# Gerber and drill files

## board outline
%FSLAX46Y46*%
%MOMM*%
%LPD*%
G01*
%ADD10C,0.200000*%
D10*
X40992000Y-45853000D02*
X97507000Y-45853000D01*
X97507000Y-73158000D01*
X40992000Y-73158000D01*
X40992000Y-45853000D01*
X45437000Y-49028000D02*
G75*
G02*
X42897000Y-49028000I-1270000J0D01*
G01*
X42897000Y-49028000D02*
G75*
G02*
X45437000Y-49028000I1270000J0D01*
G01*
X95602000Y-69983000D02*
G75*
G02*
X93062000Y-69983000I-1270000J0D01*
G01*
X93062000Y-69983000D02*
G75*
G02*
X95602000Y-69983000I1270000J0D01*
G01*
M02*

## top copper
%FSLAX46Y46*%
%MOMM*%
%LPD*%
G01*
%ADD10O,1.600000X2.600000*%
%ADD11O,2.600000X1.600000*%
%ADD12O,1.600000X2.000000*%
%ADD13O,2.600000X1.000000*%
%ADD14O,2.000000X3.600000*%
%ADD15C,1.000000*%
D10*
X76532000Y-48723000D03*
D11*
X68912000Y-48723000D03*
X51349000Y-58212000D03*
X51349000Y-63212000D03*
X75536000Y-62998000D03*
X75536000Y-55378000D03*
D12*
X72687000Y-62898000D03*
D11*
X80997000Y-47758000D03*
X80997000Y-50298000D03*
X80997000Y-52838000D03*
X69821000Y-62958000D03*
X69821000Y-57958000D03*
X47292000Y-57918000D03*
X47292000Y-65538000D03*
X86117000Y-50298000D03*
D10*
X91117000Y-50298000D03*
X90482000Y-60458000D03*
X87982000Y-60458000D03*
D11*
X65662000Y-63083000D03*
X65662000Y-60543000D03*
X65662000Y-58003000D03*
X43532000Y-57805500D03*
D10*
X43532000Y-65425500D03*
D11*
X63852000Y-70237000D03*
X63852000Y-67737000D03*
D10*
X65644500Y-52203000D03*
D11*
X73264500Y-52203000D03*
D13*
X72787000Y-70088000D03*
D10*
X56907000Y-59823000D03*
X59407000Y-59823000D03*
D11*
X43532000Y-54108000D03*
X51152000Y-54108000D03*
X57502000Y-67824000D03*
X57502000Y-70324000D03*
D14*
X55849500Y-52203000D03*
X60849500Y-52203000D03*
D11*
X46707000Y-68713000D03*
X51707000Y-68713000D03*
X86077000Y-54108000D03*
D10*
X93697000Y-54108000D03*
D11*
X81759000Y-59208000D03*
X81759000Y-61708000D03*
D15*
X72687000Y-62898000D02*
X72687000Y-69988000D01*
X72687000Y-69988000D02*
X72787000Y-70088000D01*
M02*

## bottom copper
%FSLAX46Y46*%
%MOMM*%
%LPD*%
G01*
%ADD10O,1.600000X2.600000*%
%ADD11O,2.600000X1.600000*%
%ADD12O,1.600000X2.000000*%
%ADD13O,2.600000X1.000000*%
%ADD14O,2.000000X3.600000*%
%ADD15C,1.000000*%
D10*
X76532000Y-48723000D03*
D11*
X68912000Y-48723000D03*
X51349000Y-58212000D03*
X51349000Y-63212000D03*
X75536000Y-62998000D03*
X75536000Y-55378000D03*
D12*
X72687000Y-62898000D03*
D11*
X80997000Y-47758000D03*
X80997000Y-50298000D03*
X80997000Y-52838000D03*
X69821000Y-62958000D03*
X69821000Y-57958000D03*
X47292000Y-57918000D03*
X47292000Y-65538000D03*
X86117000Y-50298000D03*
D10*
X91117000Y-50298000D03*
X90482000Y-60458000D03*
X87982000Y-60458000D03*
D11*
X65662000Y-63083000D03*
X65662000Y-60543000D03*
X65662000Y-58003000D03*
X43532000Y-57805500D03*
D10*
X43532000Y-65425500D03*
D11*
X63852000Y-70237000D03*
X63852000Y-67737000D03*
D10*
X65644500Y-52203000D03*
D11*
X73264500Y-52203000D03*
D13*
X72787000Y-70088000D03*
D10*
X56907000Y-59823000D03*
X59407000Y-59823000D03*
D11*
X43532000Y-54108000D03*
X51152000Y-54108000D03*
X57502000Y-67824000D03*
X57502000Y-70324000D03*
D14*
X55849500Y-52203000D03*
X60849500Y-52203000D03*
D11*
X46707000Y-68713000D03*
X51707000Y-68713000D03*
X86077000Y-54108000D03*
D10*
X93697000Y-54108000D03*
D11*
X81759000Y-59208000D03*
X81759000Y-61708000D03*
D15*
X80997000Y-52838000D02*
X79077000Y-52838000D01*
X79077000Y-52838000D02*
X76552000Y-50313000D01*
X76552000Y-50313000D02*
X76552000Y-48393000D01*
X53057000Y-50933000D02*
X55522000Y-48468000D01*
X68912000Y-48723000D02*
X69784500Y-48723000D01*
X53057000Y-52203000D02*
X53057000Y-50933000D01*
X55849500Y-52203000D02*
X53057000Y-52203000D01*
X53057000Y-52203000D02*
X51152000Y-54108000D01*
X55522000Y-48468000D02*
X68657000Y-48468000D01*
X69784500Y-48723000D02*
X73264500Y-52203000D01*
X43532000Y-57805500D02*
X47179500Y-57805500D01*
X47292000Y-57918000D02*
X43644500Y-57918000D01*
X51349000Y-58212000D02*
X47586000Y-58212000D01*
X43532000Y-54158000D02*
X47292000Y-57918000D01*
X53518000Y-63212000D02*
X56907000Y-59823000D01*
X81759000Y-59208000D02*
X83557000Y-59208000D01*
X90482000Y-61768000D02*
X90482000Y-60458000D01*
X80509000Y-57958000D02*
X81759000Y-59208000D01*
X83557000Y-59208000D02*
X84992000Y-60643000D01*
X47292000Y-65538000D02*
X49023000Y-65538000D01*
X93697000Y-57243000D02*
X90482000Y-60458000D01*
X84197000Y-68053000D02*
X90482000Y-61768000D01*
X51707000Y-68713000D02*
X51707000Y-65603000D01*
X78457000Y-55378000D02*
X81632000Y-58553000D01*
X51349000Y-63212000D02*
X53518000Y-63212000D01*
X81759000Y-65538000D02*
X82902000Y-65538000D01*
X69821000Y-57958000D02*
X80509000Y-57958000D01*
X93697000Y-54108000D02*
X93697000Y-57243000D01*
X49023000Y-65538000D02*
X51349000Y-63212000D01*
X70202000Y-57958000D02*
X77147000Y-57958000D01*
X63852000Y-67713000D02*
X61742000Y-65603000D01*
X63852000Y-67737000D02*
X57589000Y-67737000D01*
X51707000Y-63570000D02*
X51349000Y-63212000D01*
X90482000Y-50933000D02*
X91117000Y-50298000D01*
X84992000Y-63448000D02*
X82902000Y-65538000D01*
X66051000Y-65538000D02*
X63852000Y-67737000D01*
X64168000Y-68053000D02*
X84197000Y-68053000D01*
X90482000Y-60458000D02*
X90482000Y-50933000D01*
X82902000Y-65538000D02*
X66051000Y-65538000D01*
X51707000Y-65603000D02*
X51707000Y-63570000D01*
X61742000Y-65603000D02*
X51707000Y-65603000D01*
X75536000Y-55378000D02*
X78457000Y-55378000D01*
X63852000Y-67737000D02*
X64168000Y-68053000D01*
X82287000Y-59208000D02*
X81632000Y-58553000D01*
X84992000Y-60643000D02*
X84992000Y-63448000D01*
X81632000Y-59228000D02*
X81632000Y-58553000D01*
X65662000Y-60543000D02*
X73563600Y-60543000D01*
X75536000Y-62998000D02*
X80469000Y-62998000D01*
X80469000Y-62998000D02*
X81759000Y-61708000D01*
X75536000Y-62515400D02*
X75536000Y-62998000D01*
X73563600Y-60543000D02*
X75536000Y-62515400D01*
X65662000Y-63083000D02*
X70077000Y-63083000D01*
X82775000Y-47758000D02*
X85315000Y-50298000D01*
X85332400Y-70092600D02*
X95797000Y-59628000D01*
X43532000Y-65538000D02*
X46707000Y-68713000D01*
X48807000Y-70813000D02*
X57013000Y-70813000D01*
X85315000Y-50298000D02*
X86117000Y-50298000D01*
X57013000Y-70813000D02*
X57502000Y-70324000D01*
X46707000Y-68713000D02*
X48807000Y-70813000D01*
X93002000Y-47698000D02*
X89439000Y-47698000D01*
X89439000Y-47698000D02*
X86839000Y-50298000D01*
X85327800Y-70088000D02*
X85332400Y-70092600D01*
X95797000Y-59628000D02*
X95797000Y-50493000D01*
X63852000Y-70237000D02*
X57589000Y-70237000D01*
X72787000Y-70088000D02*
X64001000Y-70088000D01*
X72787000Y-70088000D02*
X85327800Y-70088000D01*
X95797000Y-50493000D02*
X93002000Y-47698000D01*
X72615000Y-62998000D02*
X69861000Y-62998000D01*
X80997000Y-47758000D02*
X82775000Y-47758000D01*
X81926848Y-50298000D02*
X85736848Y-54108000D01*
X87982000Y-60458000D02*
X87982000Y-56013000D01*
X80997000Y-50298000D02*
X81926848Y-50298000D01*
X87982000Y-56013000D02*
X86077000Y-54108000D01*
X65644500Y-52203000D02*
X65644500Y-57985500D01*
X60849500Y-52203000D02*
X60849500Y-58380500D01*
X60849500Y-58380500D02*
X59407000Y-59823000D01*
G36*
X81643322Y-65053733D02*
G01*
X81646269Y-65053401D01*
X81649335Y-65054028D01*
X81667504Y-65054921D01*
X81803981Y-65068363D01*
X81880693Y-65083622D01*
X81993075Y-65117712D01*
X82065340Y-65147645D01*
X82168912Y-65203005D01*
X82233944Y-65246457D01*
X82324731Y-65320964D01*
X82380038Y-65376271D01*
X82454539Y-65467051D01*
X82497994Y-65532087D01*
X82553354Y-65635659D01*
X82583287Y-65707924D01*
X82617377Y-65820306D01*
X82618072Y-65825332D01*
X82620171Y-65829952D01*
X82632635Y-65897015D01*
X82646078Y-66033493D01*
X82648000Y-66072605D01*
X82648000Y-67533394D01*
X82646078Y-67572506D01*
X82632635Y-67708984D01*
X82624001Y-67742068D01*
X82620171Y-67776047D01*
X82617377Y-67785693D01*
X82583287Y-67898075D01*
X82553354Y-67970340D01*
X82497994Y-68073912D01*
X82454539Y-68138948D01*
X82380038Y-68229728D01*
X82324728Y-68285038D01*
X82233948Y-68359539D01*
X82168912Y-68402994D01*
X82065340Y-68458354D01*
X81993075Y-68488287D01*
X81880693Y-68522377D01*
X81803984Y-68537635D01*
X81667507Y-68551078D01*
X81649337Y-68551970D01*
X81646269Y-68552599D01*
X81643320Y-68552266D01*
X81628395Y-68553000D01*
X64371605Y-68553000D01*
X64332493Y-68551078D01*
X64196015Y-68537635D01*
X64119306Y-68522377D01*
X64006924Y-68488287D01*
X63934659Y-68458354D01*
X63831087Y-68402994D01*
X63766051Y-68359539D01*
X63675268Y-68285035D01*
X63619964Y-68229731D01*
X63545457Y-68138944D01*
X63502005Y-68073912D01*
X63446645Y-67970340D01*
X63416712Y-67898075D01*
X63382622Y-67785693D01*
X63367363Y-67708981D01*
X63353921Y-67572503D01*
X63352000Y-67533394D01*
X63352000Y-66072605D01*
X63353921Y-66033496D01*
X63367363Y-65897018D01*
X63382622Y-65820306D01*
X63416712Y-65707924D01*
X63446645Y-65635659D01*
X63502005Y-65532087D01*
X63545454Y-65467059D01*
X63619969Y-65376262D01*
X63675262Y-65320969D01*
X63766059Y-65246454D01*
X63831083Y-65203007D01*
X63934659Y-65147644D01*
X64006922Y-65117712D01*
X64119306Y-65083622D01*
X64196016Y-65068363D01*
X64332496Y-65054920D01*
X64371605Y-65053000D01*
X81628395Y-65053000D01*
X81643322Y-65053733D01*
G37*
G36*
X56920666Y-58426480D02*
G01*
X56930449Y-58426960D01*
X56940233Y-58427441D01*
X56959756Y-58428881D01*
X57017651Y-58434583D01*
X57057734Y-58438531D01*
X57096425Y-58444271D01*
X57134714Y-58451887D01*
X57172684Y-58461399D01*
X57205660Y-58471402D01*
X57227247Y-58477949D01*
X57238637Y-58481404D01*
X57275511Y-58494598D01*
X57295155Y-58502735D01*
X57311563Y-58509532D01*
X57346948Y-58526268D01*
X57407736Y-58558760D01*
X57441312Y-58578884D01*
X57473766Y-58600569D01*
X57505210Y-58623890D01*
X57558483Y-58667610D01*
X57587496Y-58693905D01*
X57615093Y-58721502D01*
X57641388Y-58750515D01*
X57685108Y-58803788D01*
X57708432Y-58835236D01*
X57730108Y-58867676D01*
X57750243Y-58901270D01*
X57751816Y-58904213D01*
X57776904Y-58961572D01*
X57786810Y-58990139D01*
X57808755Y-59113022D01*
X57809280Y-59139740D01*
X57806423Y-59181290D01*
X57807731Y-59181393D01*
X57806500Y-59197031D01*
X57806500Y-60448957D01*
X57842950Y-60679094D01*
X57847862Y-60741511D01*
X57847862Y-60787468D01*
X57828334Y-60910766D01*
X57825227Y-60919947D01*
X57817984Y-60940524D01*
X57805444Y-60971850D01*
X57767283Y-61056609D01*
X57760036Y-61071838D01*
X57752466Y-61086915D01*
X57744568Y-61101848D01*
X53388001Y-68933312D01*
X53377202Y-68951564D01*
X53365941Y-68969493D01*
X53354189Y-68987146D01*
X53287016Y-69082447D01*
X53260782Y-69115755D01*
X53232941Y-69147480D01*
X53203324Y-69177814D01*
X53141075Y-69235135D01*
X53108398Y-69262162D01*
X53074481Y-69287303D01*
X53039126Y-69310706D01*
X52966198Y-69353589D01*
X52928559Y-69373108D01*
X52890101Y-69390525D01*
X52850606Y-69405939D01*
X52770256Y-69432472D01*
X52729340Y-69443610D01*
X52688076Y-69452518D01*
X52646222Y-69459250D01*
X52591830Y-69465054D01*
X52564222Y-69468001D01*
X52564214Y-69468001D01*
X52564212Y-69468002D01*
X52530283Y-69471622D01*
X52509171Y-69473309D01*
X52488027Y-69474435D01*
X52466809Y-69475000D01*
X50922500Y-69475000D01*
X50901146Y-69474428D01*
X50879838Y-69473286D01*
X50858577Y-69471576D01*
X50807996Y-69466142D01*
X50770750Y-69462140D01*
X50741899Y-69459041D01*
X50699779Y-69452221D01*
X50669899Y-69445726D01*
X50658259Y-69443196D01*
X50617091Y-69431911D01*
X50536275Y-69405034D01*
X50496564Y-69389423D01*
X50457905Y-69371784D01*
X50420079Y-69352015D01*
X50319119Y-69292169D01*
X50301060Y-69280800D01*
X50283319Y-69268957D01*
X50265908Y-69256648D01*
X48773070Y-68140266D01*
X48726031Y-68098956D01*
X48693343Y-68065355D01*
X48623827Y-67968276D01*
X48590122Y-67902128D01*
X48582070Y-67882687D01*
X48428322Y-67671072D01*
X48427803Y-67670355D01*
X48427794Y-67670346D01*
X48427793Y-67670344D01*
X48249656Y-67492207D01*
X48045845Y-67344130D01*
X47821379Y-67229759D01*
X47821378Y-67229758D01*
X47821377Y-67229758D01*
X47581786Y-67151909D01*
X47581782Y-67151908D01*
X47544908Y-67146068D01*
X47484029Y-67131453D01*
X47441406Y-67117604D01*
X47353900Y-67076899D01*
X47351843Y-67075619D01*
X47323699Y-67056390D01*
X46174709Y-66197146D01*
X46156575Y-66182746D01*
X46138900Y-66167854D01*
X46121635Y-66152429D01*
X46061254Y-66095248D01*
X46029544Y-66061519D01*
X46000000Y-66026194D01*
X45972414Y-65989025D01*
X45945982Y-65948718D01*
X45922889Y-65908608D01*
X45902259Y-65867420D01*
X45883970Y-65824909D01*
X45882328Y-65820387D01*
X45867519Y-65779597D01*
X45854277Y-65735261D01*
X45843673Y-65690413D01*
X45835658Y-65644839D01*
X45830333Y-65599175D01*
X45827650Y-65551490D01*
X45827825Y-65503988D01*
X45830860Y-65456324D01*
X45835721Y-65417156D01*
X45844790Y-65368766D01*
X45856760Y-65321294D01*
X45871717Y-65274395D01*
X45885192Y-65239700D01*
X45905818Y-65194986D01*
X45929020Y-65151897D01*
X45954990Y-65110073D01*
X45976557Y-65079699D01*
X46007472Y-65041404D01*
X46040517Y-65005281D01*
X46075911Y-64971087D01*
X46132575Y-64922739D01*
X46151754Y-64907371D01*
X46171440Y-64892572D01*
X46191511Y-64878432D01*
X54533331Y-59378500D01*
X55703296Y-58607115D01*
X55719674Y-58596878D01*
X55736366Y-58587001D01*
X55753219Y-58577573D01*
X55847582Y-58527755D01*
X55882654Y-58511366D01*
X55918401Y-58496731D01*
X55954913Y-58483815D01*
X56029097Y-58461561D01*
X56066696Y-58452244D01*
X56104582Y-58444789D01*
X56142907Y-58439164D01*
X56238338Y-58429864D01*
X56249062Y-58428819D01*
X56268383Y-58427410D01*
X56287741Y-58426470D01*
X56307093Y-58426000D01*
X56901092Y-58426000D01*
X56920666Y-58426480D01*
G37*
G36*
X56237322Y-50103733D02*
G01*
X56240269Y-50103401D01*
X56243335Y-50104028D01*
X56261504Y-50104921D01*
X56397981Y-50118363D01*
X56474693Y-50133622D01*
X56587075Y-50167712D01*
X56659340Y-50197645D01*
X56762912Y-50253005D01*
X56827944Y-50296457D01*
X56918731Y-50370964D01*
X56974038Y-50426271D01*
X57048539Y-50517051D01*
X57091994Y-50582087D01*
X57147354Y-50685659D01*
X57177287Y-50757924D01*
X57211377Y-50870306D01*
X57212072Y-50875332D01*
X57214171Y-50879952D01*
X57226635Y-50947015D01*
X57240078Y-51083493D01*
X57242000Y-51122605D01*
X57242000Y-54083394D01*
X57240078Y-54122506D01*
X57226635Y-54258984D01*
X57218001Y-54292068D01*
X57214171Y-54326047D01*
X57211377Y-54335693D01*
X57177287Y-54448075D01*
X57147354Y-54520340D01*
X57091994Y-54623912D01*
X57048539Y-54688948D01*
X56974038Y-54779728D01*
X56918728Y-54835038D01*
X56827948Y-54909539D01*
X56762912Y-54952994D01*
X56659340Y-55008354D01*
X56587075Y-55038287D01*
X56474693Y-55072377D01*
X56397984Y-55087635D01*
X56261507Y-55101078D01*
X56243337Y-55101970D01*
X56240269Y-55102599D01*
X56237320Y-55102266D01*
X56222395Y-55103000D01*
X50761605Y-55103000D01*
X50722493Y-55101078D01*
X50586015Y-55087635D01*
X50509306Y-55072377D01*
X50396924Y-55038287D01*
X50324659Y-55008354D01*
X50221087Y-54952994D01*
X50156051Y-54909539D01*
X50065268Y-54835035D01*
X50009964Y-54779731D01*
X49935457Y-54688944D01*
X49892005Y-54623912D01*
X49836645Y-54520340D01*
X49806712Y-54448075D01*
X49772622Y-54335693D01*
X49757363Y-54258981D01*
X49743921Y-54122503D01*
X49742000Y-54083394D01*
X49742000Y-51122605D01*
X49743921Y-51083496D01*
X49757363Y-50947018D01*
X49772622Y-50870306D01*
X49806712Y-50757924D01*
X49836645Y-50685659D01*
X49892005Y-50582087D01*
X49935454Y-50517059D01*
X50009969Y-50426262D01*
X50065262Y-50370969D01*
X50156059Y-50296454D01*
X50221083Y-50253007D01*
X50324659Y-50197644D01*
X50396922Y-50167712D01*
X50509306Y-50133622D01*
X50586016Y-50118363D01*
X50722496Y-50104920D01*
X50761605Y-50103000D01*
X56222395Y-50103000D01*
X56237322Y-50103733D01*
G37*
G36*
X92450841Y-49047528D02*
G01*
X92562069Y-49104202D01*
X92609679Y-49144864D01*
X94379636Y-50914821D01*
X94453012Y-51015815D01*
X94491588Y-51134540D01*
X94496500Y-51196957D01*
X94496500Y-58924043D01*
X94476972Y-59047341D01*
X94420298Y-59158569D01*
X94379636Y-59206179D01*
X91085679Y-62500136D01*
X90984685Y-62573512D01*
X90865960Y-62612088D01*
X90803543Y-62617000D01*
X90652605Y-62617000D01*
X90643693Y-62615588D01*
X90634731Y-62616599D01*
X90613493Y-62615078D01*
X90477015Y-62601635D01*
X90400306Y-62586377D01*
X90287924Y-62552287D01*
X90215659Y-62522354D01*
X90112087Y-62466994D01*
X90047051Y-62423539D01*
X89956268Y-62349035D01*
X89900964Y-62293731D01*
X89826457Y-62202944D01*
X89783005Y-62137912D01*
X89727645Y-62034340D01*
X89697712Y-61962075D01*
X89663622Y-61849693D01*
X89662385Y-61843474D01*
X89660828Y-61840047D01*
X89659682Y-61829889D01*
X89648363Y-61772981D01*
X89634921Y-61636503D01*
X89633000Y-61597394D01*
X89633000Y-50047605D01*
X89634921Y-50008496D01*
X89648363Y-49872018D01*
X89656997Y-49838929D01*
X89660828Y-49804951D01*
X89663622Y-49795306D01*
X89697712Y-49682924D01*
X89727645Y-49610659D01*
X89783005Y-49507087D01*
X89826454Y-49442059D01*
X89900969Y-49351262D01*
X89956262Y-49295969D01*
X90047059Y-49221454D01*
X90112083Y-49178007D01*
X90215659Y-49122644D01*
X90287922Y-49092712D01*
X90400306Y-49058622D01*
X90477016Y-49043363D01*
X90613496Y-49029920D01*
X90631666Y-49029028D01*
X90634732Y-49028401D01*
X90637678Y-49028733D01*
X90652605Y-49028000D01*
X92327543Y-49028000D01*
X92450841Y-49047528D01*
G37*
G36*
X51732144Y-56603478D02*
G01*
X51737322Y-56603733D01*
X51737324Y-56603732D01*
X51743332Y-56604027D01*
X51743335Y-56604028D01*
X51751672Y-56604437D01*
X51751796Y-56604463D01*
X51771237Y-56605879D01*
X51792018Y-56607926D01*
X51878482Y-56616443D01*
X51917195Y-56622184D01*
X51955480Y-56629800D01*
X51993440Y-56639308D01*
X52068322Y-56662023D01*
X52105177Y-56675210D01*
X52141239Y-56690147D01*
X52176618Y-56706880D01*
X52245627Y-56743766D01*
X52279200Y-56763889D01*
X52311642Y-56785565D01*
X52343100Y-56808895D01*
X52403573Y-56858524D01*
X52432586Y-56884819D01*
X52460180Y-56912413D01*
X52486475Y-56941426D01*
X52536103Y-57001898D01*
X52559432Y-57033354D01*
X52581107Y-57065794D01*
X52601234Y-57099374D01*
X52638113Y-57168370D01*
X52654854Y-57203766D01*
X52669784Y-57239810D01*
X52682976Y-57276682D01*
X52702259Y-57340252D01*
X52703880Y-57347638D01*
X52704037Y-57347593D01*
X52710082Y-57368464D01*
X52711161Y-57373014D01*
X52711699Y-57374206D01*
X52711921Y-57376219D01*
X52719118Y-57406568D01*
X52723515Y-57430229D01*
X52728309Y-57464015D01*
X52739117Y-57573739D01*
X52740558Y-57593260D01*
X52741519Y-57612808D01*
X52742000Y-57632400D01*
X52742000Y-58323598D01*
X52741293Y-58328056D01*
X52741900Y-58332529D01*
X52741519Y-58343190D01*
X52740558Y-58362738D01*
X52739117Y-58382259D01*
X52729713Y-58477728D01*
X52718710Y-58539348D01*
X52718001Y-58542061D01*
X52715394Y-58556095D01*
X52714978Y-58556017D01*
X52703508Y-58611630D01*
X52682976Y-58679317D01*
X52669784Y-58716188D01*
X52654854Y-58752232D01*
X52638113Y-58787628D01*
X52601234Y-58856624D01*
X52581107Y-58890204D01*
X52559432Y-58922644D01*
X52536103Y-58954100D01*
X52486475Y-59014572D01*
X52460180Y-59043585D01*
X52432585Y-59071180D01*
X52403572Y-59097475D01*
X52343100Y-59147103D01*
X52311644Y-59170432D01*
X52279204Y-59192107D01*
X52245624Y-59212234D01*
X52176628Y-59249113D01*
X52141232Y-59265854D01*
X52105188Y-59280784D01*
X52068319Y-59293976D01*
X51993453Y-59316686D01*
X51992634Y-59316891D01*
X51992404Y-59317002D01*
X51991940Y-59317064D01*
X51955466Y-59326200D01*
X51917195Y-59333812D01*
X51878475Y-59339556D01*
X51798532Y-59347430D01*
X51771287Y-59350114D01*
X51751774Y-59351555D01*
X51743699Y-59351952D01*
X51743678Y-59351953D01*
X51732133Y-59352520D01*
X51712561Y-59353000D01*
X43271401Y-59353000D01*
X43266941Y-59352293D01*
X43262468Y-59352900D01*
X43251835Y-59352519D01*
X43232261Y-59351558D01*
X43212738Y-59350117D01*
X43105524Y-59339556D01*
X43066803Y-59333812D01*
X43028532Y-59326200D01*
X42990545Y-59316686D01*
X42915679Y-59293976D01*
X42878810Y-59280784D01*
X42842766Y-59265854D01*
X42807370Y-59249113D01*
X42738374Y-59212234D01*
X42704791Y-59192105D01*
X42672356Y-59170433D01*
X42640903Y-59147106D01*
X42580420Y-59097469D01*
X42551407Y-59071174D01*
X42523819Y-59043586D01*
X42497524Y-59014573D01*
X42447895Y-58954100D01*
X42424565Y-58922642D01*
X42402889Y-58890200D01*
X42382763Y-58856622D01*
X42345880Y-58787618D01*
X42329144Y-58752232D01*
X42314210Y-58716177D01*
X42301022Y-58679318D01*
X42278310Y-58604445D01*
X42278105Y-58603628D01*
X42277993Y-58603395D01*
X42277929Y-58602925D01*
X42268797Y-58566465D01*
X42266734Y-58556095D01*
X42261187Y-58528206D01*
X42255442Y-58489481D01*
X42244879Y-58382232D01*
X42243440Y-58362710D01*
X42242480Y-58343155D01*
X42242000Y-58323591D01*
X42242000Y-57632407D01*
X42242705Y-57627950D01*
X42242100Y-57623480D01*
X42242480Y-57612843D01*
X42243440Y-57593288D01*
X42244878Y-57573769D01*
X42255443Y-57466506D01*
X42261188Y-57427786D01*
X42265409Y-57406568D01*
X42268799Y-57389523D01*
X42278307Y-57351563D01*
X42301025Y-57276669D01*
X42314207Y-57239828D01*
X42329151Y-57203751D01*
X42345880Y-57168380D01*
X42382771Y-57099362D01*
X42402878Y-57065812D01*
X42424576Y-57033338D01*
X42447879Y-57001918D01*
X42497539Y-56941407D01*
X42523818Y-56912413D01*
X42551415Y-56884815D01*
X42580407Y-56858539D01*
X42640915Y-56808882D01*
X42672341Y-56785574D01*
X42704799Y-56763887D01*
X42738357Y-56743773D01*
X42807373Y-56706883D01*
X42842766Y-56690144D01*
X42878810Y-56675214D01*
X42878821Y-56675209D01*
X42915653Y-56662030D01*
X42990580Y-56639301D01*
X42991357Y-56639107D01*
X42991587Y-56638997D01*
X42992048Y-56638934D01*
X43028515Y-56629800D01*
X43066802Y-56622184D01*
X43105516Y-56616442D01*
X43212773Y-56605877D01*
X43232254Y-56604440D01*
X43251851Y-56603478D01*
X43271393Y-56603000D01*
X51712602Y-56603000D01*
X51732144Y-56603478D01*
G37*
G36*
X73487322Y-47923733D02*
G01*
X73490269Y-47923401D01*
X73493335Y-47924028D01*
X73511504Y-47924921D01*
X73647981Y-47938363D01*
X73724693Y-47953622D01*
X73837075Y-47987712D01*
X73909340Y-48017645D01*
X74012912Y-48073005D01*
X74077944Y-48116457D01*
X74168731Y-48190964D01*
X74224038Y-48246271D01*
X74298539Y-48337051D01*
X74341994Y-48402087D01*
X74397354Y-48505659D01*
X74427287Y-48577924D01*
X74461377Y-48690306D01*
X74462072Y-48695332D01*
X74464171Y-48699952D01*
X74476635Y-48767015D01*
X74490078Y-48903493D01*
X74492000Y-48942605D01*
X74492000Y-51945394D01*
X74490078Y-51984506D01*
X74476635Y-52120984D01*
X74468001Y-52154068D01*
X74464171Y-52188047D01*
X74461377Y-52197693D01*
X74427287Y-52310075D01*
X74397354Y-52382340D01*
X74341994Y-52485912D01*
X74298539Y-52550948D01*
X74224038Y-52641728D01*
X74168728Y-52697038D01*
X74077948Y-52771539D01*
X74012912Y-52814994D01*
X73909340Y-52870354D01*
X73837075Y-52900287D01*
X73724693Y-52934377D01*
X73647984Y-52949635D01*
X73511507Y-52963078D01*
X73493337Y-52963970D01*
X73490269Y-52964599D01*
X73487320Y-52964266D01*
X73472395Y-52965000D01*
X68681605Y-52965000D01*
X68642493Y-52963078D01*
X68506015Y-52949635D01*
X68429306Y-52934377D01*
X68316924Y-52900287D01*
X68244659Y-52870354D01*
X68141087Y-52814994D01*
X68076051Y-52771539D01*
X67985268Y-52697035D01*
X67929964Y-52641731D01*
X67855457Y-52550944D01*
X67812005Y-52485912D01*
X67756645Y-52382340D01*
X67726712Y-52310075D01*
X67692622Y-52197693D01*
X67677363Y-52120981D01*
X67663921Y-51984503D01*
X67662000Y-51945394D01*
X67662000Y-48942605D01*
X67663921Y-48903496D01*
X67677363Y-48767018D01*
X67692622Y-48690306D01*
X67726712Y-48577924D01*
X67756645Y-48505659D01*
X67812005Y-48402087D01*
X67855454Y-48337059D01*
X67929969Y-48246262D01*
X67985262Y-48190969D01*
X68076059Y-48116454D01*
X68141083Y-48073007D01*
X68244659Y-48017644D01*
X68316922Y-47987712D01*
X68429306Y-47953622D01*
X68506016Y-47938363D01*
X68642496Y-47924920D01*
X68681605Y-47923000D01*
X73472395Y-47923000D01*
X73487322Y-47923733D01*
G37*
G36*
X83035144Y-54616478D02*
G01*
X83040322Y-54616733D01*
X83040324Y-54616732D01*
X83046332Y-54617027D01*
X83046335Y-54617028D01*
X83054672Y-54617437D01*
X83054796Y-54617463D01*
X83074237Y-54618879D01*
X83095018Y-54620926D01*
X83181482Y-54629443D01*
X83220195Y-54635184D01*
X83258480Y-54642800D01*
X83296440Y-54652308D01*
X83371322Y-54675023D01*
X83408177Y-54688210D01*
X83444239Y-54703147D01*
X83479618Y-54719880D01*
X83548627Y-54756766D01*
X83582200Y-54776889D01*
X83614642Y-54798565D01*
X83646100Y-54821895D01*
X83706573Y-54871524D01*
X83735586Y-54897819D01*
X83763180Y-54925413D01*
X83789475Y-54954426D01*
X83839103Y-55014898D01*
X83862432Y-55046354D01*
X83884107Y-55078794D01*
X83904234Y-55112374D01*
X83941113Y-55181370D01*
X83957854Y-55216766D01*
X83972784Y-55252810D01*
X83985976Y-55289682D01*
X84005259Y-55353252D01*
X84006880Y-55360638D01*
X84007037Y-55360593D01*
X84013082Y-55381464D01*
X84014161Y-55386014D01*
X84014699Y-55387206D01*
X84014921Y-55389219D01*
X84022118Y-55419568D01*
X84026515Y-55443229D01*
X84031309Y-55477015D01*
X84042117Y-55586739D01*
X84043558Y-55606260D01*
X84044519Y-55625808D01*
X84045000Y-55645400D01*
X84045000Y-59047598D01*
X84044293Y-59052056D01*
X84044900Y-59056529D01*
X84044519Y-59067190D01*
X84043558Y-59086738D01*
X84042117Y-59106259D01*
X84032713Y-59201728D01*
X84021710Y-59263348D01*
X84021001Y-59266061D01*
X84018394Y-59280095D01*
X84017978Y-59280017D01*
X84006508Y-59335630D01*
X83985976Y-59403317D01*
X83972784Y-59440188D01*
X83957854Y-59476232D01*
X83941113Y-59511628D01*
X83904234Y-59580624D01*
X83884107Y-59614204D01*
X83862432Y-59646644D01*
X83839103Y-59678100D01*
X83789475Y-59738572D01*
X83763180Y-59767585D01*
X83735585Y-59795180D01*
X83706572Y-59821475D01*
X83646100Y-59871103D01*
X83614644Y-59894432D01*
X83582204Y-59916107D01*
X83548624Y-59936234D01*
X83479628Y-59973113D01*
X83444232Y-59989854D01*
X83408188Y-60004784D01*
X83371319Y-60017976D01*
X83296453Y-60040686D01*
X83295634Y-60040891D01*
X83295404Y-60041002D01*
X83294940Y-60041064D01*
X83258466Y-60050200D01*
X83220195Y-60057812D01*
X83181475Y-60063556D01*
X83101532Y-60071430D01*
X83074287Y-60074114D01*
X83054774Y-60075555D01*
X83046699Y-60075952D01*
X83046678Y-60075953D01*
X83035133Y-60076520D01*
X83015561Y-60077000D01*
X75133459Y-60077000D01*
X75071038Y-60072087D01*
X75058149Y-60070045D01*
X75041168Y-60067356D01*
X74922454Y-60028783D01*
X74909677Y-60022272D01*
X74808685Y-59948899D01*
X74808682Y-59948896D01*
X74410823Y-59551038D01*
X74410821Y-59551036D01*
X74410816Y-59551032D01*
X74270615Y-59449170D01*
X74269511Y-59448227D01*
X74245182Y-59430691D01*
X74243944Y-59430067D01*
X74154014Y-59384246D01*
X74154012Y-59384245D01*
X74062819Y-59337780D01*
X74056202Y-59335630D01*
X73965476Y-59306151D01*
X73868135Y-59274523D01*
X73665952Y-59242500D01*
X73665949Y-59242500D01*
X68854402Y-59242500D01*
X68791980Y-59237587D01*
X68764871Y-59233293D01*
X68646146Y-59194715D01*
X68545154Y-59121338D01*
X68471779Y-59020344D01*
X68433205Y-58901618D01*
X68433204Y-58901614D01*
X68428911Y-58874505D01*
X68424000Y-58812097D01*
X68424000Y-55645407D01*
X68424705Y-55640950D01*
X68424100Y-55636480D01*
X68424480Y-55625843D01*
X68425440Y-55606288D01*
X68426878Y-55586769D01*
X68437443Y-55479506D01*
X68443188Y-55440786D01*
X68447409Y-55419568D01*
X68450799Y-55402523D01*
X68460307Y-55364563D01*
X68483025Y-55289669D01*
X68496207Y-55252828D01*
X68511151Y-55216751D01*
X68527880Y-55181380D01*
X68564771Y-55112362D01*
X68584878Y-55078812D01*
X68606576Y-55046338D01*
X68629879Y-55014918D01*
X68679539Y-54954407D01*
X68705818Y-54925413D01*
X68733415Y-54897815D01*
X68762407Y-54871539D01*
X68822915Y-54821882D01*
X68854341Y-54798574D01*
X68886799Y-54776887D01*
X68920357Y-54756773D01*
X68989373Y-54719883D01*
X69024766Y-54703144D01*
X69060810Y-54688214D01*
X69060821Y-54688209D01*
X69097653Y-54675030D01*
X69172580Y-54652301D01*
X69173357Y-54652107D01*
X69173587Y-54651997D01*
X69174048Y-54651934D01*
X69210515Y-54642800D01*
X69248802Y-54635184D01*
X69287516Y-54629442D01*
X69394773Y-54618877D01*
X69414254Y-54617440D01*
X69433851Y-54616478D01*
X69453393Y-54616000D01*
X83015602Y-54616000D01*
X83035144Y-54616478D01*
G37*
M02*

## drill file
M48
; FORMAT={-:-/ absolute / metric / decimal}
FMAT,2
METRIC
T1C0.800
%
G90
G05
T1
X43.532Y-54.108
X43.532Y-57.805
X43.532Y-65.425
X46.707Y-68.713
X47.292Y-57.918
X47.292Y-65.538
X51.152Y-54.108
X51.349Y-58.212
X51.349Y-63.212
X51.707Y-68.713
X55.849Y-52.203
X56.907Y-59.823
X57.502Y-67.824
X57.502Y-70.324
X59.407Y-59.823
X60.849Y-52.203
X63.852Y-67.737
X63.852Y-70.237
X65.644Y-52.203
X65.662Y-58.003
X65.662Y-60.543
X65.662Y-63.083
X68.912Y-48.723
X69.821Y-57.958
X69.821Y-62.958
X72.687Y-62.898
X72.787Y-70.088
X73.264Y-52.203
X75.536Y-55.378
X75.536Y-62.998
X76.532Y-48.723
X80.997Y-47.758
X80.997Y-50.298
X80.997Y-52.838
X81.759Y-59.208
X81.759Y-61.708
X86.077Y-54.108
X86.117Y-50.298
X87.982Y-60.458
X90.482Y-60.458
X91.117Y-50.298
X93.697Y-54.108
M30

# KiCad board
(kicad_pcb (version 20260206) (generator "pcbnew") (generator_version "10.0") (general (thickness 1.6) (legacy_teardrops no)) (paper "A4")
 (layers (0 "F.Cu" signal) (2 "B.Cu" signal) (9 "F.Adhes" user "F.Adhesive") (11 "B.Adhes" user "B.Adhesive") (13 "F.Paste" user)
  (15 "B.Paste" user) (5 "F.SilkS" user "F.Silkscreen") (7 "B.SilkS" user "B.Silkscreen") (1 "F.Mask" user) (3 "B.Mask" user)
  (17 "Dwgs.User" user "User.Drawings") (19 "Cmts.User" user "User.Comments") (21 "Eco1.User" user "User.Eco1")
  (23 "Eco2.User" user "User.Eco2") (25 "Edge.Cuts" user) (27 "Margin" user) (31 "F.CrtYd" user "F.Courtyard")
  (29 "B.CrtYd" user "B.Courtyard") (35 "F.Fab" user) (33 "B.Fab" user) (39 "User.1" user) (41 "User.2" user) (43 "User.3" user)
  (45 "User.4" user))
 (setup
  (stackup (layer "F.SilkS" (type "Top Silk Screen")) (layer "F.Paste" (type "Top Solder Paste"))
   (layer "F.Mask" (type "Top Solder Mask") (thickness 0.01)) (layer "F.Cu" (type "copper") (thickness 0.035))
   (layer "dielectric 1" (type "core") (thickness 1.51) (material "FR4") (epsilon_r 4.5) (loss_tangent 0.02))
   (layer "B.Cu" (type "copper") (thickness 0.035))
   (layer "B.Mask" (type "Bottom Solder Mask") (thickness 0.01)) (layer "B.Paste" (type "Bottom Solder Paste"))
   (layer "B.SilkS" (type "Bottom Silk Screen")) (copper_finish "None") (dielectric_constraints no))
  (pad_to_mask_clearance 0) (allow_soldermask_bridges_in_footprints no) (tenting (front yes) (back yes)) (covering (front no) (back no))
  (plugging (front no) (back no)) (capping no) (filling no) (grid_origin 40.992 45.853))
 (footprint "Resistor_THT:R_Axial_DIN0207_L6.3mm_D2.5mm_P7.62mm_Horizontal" (layer "F.Cu") (at 76.532 48.723 180)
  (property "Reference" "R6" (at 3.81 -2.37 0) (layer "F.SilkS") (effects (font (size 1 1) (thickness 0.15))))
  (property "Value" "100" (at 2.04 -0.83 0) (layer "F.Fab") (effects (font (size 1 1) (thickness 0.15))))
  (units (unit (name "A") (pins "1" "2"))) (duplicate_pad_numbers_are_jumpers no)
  (pad "1" thru_hole oval (at 0 0 180) (size 1.6 2.6) (drill 0.8) (layers "*.Cu" "*.Mask") (remove_unused_layers no) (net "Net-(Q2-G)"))
  (pad "2" thru_hole oval (at 7.62 0 270) (size 1.6 2.6) (drill 0.8) (layers "*.Cu" "*.Mask") (remove_unused_layers no) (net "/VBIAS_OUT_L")))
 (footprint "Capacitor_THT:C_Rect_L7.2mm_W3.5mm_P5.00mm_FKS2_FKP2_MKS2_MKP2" (layer "F.Cu") (at 51.349 58.212 -90)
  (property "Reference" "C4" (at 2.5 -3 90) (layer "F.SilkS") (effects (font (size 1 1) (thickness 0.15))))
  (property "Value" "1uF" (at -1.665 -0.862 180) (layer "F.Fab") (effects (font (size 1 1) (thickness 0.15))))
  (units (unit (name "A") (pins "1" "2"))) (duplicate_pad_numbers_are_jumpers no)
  (pad "1" thru_hole oval (at 0 0 270) (size 1.6 2.6) (drill 0.8) (layers "*.Cu" "*.Mask") (remove_unused_layers no) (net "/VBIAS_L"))
  (pad "2" thru_hole oval (at 5 0 270) (size 1.6 2.6) (drill 0.8) (layers "*.Cu" "*.Mask") (remove_unused_layers no) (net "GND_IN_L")))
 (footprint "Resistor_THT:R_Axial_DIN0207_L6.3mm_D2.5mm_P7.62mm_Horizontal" (layer "F.Cu") (at 75.536 62.998 90)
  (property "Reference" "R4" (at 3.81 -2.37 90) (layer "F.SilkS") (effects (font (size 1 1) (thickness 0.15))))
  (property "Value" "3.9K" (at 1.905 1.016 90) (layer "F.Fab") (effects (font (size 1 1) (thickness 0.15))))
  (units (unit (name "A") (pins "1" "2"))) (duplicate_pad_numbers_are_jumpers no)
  (pad "1" thru_hole oval (at 0 0 90) (size 1.6 2.6) (drill 0.8) (layers "*.Cu" "*.Mask") (remove_unused_layers no) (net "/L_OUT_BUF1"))
  (pad "2" thru_hole oval (at 7.62 0 90) (size 1.6 2.6) (drill 0.8) (layers "*.Cu" "*.Mask") (remove_unused_layers no) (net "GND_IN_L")))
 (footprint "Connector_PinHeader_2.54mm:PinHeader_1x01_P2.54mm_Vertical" (layer "F.Cu") (at 72.687 62.898)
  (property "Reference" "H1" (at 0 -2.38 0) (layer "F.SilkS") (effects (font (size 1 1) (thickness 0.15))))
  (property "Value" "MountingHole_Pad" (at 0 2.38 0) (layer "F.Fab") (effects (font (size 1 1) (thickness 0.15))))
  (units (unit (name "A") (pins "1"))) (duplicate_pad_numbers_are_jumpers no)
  (pad "1" thru_hole oval (at 0 0) (size 1.6 2) (drill 0.8) (layers "*.Cu") (remove_unused_layers no) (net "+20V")))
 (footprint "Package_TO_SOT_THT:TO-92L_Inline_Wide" (layer "F.Cu") (at 80.997 47.758 -90)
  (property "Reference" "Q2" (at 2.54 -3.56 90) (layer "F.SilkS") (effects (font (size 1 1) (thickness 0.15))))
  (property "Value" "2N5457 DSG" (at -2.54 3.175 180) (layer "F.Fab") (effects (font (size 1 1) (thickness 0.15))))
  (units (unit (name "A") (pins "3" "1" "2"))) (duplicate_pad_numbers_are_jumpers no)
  (pad "1" thru_hole oval (at 0 0 270) (size 1.6 2.6) (drill 0.8) (layers "*.Cu" "*.Mask") (remove_unused_layers no) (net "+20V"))
  (pad "2" thru_hole oval (at 2.54 0 270) (size 1.6 2.6) (drill 0.8) (layers "*.Cu" "*.Mask") (remove_unused_layers no) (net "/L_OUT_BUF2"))
  (pad "3" thru_hole oval (at 5.08 0 270) (size 1.6 2.6) (drill 0.8) (layers "*.Cu" "*.Mask") (remove_unused_layers no) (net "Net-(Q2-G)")))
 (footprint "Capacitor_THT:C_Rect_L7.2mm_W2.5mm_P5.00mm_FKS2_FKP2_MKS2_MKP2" (layer "F.Cu") (at 69.821 62.958 90)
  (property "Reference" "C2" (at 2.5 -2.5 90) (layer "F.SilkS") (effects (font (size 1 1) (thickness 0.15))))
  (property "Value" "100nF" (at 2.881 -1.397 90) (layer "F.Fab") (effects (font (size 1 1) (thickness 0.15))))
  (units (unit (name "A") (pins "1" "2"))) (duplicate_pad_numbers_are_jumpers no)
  (pad "1" thru_hole oval (at 0 0 90) (size 1.6 2.6) (drill 0.8) (layers "*.Cu" "*.Mask") (remove_unused_layers no) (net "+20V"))
  (pad "2" thru_hole oval (at 5 0 90) (size 1.6 2.6) (drill 0.8) (layers "*.Cu" "*.Mask") (remove_unused_layers no) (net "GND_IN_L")))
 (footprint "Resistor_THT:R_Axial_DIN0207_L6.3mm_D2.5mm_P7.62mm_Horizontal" (layer "F.Cu") (at 47.292 57.918 -90)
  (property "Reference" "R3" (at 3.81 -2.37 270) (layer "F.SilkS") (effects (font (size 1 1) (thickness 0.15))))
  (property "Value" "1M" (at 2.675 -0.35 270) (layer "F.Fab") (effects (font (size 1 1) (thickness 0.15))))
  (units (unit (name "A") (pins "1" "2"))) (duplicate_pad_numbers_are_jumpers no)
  (pad "1" thru_hole oval (at 0 0 270) (size 1.6 2.6) (drill 0.8) (layers "*.Cu" "*.Mask") (remove_unused_layers no) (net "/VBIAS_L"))
  (pad "2" thru_hole oval (at 7.62 0 270) (size 1.6 2.6) (drill 0.8) (layers "*.Cu" "*.Mask") (remove_unused_layers no) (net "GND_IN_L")))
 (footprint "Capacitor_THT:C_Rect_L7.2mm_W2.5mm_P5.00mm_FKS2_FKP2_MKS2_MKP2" (layer "F.Cu") (at 86.117 50.298)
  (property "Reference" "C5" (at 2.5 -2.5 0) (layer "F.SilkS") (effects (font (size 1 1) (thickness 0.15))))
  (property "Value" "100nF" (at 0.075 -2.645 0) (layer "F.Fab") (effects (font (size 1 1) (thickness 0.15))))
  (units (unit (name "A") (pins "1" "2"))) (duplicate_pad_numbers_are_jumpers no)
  (pad "1" thru_hole oval (at 0 0 90) (size 1.6 2.6) (drill 0.8) (layers "*.Cu" "*.Mask") (remove_unused_layers no) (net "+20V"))
  (pad "2" thru_hole oval (at 5 0) (size 1.6 2.6) (drill 0.8) (layers "*.Cu" "*.Mask") (remove_unused_layers no) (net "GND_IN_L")))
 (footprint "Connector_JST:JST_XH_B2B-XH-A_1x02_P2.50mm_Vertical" (layer "F.Cu") (at 90.482 60.458 180)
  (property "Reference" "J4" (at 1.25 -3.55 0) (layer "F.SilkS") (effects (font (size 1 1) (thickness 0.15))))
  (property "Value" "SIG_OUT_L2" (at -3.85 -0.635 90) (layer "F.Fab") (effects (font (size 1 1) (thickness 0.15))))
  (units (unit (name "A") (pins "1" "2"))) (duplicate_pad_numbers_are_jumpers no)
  (pad "1" thru_hole oval (at 0 0 180) (size 1.6 2.6) (drill 0.8) (layers "*.Cu" "*.Mask") (remove_unused_layers no) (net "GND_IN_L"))
  (pad "2" thru_hole oval (at 2.5 0 180) (size 1.6 2.6) (drill 0.8) (layers "*.Cu" "*.Mask") (remove_unused_layers no) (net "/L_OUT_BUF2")))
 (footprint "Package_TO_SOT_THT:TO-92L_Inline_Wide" (layer "F.Cu") (at 65.662 63.083 90)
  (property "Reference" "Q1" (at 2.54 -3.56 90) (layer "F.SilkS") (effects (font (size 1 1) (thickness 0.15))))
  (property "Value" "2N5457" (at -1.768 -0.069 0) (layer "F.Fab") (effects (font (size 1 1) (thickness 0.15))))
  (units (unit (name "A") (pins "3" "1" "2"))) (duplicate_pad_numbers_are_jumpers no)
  (pad "1" thru_hole oval (at 0 0 90) (size 1.6 2.6) (drill 0.8) (layers "*.Cu" "*.Mask") (remove_unused_layers no) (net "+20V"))
  (pad "2" thru_hole oval (at 2.54 0 90) (size 1.6 2.6) (drill 0.8) (layers "*.Cu" "*.Mask") (remove_unused_layers no) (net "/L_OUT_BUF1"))
  (pad "3" thru_hole oval (at 5.08 0 90) (size 1.6 2.6) (drill 0.8) (layers "*.Cu" "*.Mask") (remove_unused_layers no) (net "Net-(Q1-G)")))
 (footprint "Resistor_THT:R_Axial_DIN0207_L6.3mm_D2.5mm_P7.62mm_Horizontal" (layer "F.Cu") (at 43.532 57.8055 -90)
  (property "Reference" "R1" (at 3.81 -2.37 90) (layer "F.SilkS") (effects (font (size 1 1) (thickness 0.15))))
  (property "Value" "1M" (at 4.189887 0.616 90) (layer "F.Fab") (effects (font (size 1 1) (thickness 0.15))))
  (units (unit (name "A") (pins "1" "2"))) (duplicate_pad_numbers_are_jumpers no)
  (pad "1" thru_hole oval (at 0 0 270) (size 1.6 2.6) (drill 0.8) (layers "*.Cu" "*.Mask") (remove_unused_layers no) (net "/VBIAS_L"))
  (pad "2" thru_hole oval (at 7.62 0) (size 1.6 2.6) (drill 0.8) (layers "*.Cu" "*.Mask") (remove_unused_layers no) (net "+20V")))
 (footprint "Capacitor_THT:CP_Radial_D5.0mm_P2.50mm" (layer "F.Cu") (at 63.852 70.237 90)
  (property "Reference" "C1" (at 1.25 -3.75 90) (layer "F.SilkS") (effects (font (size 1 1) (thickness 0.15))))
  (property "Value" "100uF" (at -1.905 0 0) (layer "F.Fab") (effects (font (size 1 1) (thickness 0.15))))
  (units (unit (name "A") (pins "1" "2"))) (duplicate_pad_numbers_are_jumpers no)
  (pad "1" thru_hole oval (at 0 0 90) (size 1.6 2.6) (drill 0.8) (layers "*.Cu" "*.Mask") (remove_unused_layers no) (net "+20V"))
  (pad "2" thru_hole oval (at 2.5 0 90) (size 1.6 2.6) (drill 0.8) (layers "*.Cu" "*.Mask") (remove_unused_layers no) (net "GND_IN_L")))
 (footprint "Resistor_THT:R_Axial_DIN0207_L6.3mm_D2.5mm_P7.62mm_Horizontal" (layer "F.Cu") (at 65.6445 52.203)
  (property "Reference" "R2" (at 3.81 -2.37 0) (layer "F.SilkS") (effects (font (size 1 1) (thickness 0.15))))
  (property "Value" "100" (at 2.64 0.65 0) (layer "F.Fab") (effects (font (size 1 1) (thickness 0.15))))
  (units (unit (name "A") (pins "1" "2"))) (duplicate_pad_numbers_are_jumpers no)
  (pad "1" thru_hole oval (at 0 0) (size 1.6 2.6) (drill 0.8) (layers "*.Cu" "*.Mask") (remove_unused_layers no) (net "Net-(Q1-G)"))
  (pad "2" thru_hole oval (at 7.62 0 90) (size 1.6 2.6) (drill 0.8) (layers "*.Cu" "*.Mask") (remove_unused_layers no) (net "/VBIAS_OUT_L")))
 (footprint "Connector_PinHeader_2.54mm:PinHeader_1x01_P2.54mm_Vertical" (layer "F.Cu") (at 72.787 70.088)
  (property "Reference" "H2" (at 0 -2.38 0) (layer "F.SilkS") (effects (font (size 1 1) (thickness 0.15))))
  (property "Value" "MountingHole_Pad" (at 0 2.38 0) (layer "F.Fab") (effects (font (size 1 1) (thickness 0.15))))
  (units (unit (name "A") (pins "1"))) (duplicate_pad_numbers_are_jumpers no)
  (pad "1" thru_hole oval (at 0 0 90) (size 1 2.6) (drill 0.8) (layers "*.Cu" "*.Mask") (remove_unused_layers no) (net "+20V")))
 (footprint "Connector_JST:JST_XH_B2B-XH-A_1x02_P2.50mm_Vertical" (layer "F.Cu") (at 56.907 59.823)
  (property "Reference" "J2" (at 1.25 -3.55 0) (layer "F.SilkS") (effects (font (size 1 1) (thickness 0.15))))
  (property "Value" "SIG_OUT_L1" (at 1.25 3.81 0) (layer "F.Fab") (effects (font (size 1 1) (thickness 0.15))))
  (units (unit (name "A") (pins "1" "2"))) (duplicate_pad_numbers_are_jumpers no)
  (pad "1" thru_hole oval (at 0 0) (size 1.6 2.6) (drill 0.8) (layers "*.Cu" "*.Mask") (remove_unused_layers no) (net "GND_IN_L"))
  (pad "2" thru_hole oval (at 2.5 0) (size 1.6 2.6) (drill 0.8) (layers "*.Cu" "*.Mask") (remove_unused_layers no) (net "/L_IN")))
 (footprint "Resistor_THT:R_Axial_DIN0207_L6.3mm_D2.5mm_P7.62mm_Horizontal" (layer "F.Cu") (at 43.532 54.108)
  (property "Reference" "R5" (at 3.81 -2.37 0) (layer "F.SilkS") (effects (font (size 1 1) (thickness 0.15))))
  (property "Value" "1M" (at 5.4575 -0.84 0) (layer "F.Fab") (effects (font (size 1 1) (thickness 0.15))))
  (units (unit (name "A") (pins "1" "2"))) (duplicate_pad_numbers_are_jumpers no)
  (pad "1" thru_hole oval (at 0 0 90) (size 1.6 2.6) (drill 0.8) (layers "*.Cu" "*.Mask") (remove_unused_layers no) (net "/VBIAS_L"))
  (pad "2" thru_hole oval (at 7.62 0 90) (size 1.6 2.6) (drill 0.8) (layers "*.Cu" "*.Mask") (remove_unused_layers no) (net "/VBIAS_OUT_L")))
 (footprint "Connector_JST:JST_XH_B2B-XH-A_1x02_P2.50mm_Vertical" (layer "F.Cu") (at 57.502 67.824 -90)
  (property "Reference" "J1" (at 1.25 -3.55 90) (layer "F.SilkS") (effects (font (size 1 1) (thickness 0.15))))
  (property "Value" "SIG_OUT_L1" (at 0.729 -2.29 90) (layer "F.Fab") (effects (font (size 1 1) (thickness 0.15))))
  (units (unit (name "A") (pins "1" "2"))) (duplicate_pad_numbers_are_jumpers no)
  (pad "1" thru_hole oval (at 0 0 270) (size 1.6 2.6) (drill 0.8) (layers "*.Cu" "*.Mask") (remove_unused_layers no) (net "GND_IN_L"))
  (pad "2" thru_hole oval (at 2.5 0 270) (size 1.6 2.6) (drill 0.8) (layers "*.Cu" "*.Mask") (remove_unused_layers no) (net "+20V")))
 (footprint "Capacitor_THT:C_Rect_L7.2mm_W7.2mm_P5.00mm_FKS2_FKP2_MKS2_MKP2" (layer "F.Cu") (at 55.8495 52.203)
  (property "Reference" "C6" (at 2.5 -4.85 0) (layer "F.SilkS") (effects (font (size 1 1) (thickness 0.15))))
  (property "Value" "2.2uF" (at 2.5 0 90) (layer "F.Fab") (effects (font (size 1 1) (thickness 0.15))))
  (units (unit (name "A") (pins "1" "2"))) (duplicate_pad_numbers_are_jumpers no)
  (pad "1" thru_hole oval (at 0 0) (size 2 3.6) (drill 0.8) (layers "*.Cu" "*.Mask") (remove_unused_layers no) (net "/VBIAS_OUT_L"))
  (pad "2" thru_hole oval (at 5 0) (size 2 3.6) (drill 0.8) (layers "*.Cu" "*.Mask") (remove_unused_layers no) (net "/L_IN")))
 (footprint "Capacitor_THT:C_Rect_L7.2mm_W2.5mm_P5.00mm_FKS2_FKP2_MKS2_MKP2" (layer "F.Cu") (at 46.707 68.713)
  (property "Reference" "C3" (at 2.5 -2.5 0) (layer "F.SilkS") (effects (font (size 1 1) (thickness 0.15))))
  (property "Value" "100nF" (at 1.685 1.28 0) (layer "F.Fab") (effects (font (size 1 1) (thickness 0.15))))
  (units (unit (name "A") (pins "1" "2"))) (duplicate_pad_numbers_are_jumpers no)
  (pad "1" thru_hole oval (at 0 0 90) (size 1.6 2.6) (drill 0.8) (layers "*.Cu" "*.Mask") (remove_unused_layers no) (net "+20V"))
  (pad "2" thru_hole oval (at 5 0 90) (size 1.6 2.6) (drill 0.8) (layers "*.Cu" "*.Mask") (remove_unused_layers no) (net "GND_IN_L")))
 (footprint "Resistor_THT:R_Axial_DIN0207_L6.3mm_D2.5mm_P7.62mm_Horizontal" (layer "F.Cu") (at 86.077 54.108)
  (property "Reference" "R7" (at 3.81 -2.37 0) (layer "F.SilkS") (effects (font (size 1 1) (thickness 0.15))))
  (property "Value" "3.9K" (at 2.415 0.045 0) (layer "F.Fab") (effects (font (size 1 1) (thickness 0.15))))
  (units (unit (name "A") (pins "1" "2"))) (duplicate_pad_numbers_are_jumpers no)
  (pad "1" thru_hole oval (at 0 0 90) (size 1.6 2.6) (drill 0.8) (layers "*.Cu" "*.Mask") (remove_unused_layers no) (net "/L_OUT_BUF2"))
  (pad "2" thru_hole oval (at 7.62 0) (size 1.6 2.6) (drill 0.8) (layers "*.Cu" "*.Mask") (remove_unused_layers no) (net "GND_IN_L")))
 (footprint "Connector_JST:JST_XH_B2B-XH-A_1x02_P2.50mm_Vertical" (layer "F.Cu") (at 81.759 59.208 -90)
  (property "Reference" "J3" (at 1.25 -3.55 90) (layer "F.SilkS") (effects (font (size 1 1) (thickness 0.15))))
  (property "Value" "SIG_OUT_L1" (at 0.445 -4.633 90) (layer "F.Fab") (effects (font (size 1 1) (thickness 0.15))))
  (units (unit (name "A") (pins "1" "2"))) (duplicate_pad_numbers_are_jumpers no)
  (pad "1" thru_hole oval (at 0 0 270) (size 1.6 2.6) (drill 0.8) (layers "*.Cu" "*.Mask") (remove_unused_layers no) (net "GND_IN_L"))
  (pad "2" thru_hole oval (at 2.5 0 270) (size 1.6 2.6) (drill 0.8) (layers "*.Cu" "*.Mask") (remove_unused_layers no) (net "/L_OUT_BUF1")))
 (gr_rect (start 40.992 45.853) (end 97.507 73.158) (stroke (width 0.2) (type solid)) (fill no) (layer "Edge.Cuts"))
 (gr_circle (center 44.167 49.028) (end 42.897 49.028) (stroke (width 0.2) (type solid)) (fill no) (layer "Edge.Cuts"))
 (gr_circle (center 94.332 69.983) (end 93.062 69.983) (stroke (width 0.2) (type solid)) (fill no) (layer "Edge.Cuts"))
 (segment (start 80.997 52.838) (end 79.077 52.838) (width 1) (layer "B.Cu") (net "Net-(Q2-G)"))
 (segment (start 79.077 52.838) (end 76.552 50.313) (width 1) (layer "B.Cu") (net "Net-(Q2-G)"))
 (segment (start 76.552 50.313) (end 76.552 48.393) (width 1) (layer "B.Cu") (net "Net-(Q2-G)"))
 (segment (start 53.057 50.933) (end 55.522 48.468) (width 1) (layer "B.Cu") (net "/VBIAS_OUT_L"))
 (segment (start 68.912 48.723) (end 69.7845 48.723) (width 1) (layer "B.Cu") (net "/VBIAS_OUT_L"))
 (segment (start 53.057 52.203) (end 53.057 50.933) (width 1) (layer "B.Cu") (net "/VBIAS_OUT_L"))
 (segment (start 55.8495 52.203) (end 53.057 52.203) (width 1) (layer "B.Cu") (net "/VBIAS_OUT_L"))
 (segment (start 53.057 52.203) (end 51.152 54.108) (width 1) (layer "B.Cu") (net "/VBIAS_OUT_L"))
 (segment (start 55.522 48.468) (end 68.657 48.468) (width 1) (layer "B.Cu") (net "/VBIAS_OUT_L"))
 (segment (start 69.7845 48.723) (end 73.2645 52.203) (width 1) (layer "B.Cu") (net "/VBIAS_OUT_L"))
 (segment (start 43.532 57.8055) (end 47.1795 57.8055) (width 1) (layer "B.Cu") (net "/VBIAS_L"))
 (segment (start 47.292 57.918) (end 43.6445 57.918) (width 1) (layer "B.Cu") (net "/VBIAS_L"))
 (segment (start 51.349 58.212) (end 47.586 58.212) (width 1) (layer "B.Cu") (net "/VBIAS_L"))
 (segment (start 43.532 54.158) (end 47.292 57.918) (width 1) (layer "B.Cu") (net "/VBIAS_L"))
 (segment (start 53.518 63.212) (end 56.907 59.823) (width 1) (layer "B.Cu") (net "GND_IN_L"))
 (segment (start 81.759 59.208) (end 83.557 59.208) (width 1) (layer "B.Cu") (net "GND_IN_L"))
 (segment (start 90.482 61.768) (end 90.482 60.458) (width 1) (layer "B.Cu") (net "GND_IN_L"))
 (segment (start 80.509 57.958) (end 81.759 59.208) (width 1) (layer "B.Cu") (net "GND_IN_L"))
 (segment (start 83.557 59.208) (end 84.992 60.643) (width 1) (layer "B.Cu") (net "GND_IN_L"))
 (segment (start 47.292 65.538) (end 49.023 65.538) (width 1) (layer "B.Cu") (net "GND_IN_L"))
 (segment (start 93.697 57.243) (end 90.482 60.458) (width 1) (layer "B.Cu") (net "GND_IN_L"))
 (segment (start 84.197 68.053) (end 90.482 61.768) (width 1) (layer "B.Cu") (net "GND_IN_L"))
 (segment (start 51.707 68.713) (end 51.707 65.603) (width 1) (layer "B.Cu") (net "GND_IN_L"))
 (segment (start 78.457 55.378) (end 81.632 58.553) (width 1) (layer "B.Cu") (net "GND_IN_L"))
 (segment (start 51.349 63.212) (end 53.518 63.212) (width 1) (layer "B.Cu") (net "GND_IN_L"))
 (segment (start 81.759 65.538) (end 82.902 65.538) (width 1) (layer "B.Cu") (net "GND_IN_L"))
 (segment (start 69.821 57.958) (end 80.509 57.958) (width 1) (layer "B.Cu") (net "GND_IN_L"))
 (segment (start 93.697 54.108) (end 93.697 57.243) (width 1) (layer "B.Cu") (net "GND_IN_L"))
 (segment (start 49.023 65.538) (end 51.349 63.212) (width 1) (layer "B.Cu") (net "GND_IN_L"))
 (segment (start 70.202 57.958) (end 77.147 57.958) (width 1) (layer "B.Cu") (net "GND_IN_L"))
 (segment (start 63.852 67.713) (end 61.742 65.603) (width 1) (layer "B.Cu") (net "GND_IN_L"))
 (segment (start 63.852 67.737) (end 57.589 67.737) (width 1) (layer "B.Cu") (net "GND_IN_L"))
 (segment (start 51.707 63.57) (end 51.349 63.212) (width 1) (layer "B.Cu") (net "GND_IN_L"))
 (segment (start 90.482 50.933) (end 91.117 50.298) (width 1) (layer "B.Cu") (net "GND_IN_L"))
 (segment (start 84.992 63.448) (end 82.902 65.538) (width 1) (layer "B.Cu") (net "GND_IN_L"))
 (segment (start 66.051 65.538) (end 63.852 67.737) (width 1) (layer "B.Cu") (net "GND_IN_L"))
 (segment (start 64.168 68.053) (end 84.197 68.053) (width 1) (layer "B.Cu") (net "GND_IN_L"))
 (segment (start 90.482 60.458) (end 90.482 50.933) (width 1) (layer "B.Cu") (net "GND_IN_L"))
 (segment (start 82.902 65.538) (end 66.051 65.538) (width 1) (layer "B.Cu") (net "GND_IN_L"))
 (segment (start 51.707 65.603) (end 51.707 63.57) (width 1) (layer "B.Cu") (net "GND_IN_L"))
 (segment (start 61.742 65.603) (end 51.707 65.603) (width 1) (layer "B.Cu") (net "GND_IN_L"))
 (segment (start 75.536 55.378) (end 78.457 55.378) (width 1) (layer "B.Cu") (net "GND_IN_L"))
 (segment (start 63.852 67.737) (end 64.168 68.053) (width 1) (layer "B.Cu") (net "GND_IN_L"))
 (segment (start 82.287 59.208) (end 81.632 58.553) (width 1) (layer "B.Cu") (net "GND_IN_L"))
 (segment (start 84.992 60.643) (end 84.992 63.448) (width 1) (layer "B.Cu") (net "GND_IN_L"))
 (segment (start 81.632 59.228) (end 81.632 58.553) (width 1) (layer "B.Cu") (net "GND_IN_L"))
 (segment (start 65.662 60.543) (end 73.5636 60.543) (width 1) (layer "B.Cu") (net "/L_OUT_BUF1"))
 (segment (start 75.536 62.998) (end 80.469 62.998) (width 1) (layer "B.Cu") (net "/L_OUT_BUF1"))
 (segment (start 80.469 62.998) (end 81.759 61.708) (width 1) (layer "B.Cu") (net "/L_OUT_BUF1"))
 (segment (start 75.536 62.5154) (end 75.536 62.998) (width 1) (layer "B.Cu") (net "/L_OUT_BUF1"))
 (segment (start 73.5636 60.543) (end 75.536 62.5154) (width 1) (layer "B.Cu") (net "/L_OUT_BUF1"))
 (segment (start 72.687 62.898) (end 72.687 69.988) (width 1) (layer "F.Cu") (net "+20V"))
 (segment (start 72.687 69.988) (end 72.787 70.088) (width 1) (layer "F.Cu") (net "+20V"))
 (segment (start 65.662 63.083) (end 70.077 63.083) (width 1) (layer "B.Cu") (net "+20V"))
 (segment (start 82.775 47.758) (end 85.315 50.298) (width 1) (layer "B.Cu") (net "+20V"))
 (segment (start 85.3324 70.0926) (end 95.797 59.628) (width 1) (layer "B.Cu") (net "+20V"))
 (segment (start 43.532 65.538) (end 46.707 68.713) (width 1) (layer "B.Cu") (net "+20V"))
 (segment (start 48.807 70.813) (end 57.013 70.813) (width 1) (layer "B.Cu") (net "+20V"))
 (segment (start 85.315 50.298) (end 86.117 50.298) (width 1) (layer "B.Cu") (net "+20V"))
 (segment (start 57.013 70.813) (end 57.502 70.324) (width 1) (layer "B.Cu") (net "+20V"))
 (segment (start 46.707 68.713) (end 48.807 70.813) (width 1) (layer "B.Cu") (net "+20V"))
 (segment (start 93.002 47.698) (end 89.439 47.698) (width 1) (layer "B.Cu") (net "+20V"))
 (segment (start 89.439 47.698) (end 86.839 50.298) (width 1) (layer "B.Cu") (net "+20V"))
 (segment (start 85.3278 70.088) (end 85.3324 70.0926) (width 1) (layer "B.Cu") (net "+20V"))
 (segment (start 95.797 59.628) (end 95.797 50.493) (width 1) (layer "B.Cu") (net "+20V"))
 (segment (start 63.852 70.237) (end 57.589 70.237) (width 1) (layer "B.Cu") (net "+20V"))
 (segment (start 72.787 70.088) (end 64.001 70.088) (width 1) (layer "B.Cu") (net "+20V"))
 (segment (start 72.787 70.088) (end 85.3278 70.088) (width 1) (layer "B.Cu") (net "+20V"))
 (segment (start 95.797 50.493) (end 93.002 47.698) (width 1) (layer "B.Cu") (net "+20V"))
 (segment (start 72.615 62.998) (end 69.861 62.998) (width 1) (layer "B.Cu") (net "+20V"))
 (segment (start 80.997 47.758) (end 82.775 47.758) (width 1) (layer "B.Cu") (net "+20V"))
 (segment (start 81.926848 50.298) (end 85.736848 54.108) (width 1) (layer "B.Cu") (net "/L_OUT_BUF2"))
 (segment (start 87.982 60.458) (end 87.982 56.013) (width 1) (layer "B.Cu") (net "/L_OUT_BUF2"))
 (segment (start 80.997 50.298) (end 81.926848 50.298) (width 1) (layer "B.Cu") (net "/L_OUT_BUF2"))
 (segment (start 87.982 56.013) (end 86.077 54.108) (width 1) (layer "B.Cu") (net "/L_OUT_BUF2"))
 (segment (start 65.6445 52.203) (end 65.6445 57.9855) (width 1) (layer "B.Cu") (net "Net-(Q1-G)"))
 (segment (start 60.8495 52.203) (end 60.8495 58.3805) (width 1) (layer "B.Cu") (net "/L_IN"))
 (segment (start 60.8495 58.3805) (end 59.407 59.823) (width 1) (layer "B.Cu") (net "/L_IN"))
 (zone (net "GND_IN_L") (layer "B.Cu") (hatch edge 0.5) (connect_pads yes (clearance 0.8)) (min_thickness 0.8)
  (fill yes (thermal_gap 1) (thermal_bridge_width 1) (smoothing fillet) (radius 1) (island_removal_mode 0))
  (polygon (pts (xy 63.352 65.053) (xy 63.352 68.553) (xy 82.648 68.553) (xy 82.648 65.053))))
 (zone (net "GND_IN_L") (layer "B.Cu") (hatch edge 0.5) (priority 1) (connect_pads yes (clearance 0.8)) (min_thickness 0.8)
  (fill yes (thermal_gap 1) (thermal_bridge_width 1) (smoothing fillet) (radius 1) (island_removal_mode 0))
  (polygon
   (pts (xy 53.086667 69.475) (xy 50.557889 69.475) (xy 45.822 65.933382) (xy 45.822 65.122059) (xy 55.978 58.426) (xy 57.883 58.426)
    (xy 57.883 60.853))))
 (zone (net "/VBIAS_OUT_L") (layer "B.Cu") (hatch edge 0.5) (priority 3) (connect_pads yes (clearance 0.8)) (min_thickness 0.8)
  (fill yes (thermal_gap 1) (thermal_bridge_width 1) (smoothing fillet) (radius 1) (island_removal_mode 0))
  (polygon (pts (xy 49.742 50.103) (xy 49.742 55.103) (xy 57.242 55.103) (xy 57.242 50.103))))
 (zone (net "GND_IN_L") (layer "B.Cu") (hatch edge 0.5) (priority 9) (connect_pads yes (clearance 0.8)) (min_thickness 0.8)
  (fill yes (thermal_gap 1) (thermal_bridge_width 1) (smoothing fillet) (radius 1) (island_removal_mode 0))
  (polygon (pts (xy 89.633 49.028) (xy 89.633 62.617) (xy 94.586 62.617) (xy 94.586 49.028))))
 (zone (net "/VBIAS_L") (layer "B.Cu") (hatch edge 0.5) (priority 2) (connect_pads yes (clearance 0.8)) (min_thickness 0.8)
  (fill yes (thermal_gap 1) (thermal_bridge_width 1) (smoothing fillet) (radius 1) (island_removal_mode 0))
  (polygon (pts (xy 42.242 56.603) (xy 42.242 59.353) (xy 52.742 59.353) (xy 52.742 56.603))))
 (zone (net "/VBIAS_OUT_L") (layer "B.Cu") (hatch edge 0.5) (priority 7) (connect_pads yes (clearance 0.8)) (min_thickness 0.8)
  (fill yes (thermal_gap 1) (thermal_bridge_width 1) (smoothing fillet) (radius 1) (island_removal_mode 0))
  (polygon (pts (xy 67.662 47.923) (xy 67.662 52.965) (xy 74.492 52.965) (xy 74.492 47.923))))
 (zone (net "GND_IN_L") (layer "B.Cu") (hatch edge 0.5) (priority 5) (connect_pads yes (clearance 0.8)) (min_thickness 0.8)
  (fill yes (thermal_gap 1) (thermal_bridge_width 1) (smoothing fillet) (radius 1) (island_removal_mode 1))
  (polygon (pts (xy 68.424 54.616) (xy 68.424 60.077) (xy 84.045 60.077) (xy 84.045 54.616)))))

